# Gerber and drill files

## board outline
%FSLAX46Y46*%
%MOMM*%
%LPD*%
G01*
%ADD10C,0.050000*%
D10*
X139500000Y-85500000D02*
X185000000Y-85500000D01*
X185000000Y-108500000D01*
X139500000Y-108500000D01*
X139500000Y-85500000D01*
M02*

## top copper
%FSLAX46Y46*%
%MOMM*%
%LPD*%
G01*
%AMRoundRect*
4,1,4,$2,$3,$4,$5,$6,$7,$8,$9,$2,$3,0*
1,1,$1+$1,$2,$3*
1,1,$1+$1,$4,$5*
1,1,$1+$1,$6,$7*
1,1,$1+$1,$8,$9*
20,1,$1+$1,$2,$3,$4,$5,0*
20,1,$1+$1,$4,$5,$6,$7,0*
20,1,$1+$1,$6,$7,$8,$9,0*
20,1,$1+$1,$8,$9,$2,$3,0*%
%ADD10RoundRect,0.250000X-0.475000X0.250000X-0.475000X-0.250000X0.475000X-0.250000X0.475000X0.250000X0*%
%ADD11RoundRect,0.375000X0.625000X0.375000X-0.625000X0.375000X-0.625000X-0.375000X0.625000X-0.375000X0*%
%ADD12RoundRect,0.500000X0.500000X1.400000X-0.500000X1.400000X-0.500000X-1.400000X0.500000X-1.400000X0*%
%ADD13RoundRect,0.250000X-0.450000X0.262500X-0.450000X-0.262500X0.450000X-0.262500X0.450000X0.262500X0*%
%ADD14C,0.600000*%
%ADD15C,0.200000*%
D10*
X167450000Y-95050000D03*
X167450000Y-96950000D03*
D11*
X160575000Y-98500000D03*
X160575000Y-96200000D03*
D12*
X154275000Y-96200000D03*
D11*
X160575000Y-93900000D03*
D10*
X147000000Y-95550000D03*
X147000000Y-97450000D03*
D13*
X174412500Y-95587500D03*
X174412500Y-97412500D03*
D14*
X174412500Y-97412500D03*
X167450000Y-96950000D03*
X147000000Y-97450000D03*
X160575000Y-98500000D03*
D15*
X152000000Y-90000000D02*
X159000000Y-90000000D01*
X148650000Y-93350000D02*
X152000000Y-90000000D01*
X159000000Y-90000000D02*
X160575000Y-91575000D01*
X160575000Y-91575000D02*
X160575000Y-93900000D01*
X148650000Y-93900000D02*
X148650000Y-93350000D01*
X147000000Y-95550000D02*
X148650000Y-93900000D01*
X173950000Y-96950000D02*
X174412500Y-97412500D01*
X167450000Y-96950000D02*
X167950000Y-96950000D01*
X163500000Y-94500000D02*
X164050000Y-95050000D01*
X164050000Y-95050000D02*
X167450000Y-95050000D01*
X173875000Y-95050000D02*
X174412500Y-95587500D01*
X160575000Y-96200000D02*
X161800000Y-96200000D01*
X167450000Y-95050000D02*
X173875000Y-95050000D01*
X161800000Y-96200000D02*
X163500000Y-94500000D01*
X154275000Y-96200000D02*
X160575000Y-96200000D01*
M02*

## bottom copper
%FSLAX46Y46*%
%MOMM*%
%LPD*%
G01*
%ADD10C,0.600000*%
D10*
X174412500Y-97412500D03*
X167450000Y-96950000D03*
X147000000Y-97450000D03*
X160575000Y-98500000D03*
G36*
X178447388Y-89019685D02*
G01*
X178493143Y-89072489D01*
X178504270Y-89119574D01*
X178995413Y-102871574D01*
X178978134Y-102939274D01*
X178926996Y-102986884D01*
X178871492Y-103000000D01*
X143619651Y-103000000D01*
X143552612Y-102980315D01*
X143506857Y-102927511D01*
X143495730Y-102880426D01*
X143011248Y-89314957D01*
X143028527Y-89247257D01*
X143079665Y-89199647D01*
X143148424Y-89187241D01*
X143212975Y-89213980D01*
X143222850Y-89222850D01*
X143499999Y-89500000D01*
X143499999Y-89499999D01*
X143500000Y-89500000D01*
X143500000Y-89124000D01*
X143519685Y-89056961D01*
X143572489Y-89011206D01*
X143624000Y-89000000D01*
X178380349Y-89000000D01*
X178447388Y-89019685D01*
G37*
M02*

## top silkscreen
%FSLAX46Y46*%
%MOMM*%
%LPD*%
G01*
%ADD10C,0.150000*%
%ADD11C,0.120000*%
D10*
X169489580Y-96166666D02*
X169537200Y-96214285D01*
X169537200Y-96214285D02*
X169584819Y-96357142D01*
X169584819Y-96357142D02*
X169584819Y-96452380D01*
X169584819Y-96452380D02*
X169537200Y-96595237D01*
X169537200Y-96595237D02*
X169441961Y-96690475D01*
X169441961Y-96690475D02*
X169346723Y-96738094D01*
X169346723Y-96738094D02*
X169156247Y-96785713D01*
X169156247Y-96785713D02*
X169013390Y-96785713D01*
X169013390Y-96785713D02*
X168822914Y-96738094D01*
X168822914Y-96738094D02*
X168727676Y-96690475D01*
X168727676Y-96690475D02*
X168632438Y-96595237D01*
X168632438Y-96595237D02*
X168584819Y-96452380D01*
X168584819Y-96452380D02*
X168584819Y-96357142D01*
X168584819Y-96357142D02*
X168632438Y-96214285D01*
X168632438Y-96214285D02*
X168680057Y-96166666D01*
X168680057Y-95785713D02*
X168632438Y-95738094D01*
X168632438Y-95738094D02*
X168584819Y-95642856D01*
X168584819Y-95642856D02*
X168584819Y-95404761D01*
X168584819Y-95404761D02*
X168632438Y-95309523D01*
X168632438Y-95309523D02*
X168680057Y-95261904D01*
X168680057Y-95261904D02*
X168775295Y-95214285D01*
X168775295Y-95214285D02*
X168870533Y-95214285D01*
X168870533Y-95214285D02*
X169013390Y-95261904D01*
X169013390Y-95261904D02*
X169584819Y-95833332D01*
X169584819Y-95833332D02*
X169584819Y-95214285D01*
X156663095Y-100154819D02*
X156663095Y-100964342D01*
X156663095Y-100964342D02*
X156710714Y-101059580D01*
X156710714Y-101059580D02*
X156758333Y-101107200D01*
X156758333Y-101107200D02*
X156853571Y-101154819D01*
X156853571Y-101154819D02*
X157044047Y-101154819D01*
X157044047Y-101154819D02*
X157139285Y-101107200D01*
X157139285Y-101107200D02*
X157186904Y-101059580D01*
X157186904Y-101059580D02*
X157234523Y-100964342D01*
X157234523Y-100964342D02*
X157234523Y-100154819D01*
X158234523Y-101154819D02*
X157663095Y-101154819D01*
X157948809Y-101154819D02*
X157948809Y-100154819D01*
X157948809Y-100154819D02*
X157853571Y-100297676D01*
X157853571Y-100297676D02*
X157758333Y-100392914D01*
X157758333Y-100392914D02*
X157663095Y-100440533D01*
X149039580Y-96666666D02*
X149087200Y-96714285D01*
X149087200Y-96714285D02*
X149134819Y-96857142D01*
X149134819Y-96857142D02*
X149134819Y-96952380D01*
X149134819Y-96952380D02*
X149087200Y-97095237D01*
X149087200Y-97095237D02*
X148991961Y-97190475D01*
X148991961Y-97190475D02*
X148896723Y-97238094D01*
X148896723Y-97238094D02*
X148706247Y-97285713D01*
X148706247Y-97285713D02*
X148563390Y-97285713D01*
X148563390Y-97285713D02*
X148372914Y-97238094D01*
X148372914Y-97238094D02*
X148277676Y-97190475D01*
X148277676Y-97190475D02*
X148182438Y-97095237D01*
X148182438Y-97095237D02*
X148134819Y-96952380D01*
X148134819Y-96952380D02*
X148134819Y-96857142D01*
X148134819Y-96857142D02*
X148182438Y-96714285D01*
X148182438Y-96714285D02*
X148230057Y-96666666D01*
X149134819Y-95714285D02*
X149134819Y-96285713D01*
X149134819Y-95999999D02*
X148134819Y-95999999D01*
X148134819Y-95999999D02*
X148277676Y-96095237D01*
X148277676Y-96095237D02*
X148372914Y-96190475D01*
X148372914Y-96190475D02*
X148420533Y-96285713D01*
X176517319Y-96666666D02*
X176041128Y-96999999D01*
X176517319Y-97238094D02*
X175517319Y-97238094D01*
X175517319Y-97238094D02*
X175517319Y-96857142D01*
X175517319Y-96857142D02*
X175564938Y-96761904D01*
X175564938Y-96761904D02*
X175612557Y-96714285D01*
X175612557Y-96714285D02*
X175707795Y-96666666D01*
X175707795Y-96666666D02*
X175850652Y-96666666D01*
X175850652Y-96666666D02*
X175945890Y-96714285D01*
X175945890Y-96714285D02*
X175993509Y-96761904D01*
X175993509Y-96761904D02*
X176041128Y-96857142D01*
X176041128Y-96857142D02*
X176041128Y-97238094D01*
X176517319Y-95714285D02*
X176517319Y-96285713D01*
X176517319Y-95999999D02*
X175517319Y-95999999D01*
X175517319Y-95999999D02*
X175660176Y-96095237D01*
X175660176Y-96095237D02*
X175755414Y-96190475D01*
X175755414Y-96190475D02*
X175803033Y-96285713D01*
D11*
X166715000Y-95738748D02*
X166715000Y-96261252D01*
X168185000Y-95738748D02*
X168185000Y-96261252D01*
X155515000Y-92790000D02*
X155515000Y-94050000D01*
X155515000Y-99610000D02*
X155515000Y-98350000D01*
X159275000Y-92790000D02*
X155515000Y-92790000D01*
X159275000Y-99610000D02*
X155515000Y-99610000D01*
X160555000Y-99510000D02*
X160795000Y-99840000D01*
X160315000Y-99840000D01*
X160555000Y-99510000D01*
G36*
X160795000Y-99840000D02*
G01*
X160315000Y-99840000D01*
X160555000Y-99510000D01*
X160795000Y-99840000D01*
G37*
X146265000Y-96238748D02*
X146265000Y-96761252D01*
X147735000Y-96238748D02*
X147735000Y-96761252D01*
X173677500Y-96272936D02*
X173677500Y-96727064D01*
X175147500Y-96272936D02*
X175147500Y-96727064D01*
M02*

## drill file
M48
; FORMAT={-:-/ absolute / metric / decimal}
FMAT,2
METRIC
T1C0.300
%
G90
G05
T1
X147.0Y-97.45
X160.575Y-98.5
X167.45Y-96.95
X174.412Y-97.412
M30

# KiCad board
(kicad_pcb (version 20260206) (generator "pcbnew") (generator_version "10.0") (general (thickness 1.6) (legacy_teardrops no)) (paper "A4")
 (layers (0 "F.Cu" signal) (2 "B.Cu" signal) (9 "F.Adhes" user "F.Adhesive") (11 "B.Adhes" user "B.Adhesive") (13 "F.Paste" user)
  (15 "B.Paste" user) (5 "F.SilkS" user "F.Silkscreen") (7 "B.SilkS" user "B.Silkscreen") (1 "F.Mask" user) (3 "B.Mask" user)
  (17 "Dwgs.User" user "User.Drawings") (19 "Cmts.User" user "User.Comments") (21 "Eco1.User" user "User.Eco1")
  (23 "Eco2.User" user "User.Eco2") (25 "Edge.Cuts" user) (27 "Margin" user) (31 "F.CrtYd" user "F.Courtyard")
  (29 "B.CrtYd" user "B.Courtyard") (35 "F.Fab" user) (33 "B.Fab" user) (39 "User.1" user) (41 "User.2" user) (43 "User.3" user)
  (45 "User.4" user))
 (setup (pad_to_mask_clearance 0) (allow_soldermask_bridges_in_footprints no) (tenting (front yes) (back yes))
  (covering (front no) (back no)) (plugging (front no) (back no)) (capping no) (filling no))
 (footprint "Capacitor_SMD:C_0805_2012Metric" (layer "F.Cu") (at 167.45 96 -90)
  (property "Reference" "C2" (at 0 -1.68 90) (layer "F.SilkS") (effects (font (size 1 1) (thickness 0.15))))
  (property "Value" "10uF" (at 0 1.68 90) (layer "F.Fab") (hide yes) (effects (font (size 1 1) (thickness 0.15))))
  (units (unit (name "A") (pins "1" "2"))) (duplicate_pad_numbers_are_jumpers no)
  (fp_line (start -0.261252 0.735) (end 0.261252 0.735) (stroke (width 0.12) (type solid)) (layer "F.SilkS"))
  (fp_line (start -0.261252 -0.735) (end 0.261252 -0.735) (stroke (width 0.12) (type solid)) (layer "F.SilkS"))
  (pad "1" smd roundrect (at -0.95 0 270) (size 1 1.45) (layers "F.Cu" "F.Mask" "F.Paste") (roundrect_rratio 0.25) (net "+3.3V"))
  (pad "2" smd roundrect (at 0.95 0 270) (size 1 1.45) (layers "F.Cu" "F.Mask" "F.Paste") (roundrect_rratio 0.25) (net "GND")))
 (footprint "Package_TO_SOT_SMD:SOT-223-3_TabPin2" (layer "F.Cu") (at 157.425 96.2 180)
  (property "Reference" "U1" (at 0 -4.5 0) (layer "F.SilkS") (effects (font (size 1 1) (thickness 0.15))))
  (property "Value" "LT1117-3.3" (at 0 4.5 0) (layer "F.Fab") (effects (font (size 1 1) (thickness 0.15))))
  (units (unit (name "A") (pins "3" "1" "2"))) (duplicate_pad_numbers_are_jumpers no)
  (fp_line (start 1.91 3.41) (end 1.91 2.15) (stroke (width 0.12) (type solid)) (layer "F.SilkS"))
  (fp_line (start 1.91 -3.41) (end 1.91 -2.15) (stroke (width 0.12) (type solid)) (layer "F.SilkS"))
  (fp_line (start -1.85 3.41) (end 1.91 3.41) (stroke (width 0.12) (type solid)) (layer "F.SilkS"))
  (fp_line (start -1.85 -3.41) (end 1.91 -3.41) (stroke (width 0.12) (type solid)) (layer "F.SilkS"))
  (fp_poly
   (pts (xy -3.13 -3.31) (xy -3.37 -3.64) (xy -2.89 -3.64) (xy -3.13 -3.31)) (stroke (width 0.12) (type solid)) (fill yes) (layer "F.SilkS"))
  (pad "1" smd roundrect (at -3.15 -2.3 180) (size 2 1.5) (layers "F.Cu" "F.Mask" "F.Paste") (roundrect_rratio 0.25) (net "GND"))
  (pad "2" smd roundrect (at -3.15 0 180) (size 2 1.5) (layers "F.Cu" "F.Mask" "F.Paste") (roundrect_rratio 0.25) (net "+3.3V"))
  (pad "2" smd roundrect (at 3.15 0 180) (size 2 3.8) (layers "F.Cu" "F.Mask" "F.Paste") (roundrect_rratio 0.25) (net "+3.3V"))
  (pad "3" smd roundrect (at -3.15 2.3 180) (size 2 1.5) (layers "F.Cu" "F.Mask" "F.Paste") (roundrect_rratio 0.25) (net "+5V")))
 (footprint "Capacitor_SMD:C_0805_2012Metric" (layer "F.Cu") (at 147 96.5 -90)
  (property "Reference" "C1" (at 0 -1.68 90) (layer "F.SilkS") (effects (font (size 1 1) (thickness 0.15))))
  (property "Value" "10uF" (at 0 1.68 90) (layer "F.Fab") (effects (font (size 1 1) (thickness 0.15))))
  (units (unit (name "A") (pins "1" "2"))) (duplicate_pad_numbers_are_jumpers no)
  (fp_line (start -0.261252 0.735) (end 0.261252 0.735) (stroke (width 0.12) (type solid)) (layer "F.SilkS"))
  (fp_line (start -0.261252 -0.735) (end 0.261252 -0.735) (stroke (width 0.12) (type solid)) (layer "F.SilkS"))
  (pad "1" smd roundrect (at -0.95 0 270) (size 1 1.45) (layers "F.Cu" "F.Mask" "F.Paste") (roundrect_rratio 0.25) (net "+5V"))
  (pad "2" smd roundrect (at 0.95 0 270) (size 1 1.45) (layers "F.Cu" "F.Mask" "F.Paste") (roundrect_rratio 0.25) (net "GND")))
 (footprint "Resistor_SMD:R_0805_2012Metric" (layer "F.Cu") (at 174.4125 96.5 -90)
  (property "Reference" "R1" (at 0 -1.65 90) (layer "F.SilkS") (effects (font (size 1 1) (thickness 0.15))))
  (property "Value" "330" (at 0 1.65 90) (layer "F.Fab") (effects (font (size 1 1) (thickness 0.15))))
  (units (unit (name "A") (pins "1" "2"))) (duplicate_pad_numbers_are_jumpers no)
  (fp_line (start -0.227064 0.735) (end 0.227064 0.735) (stroke (width 0.12) (type solid)) (layer "F.SilkS"))
  (fp_line (start -0.227064 -0.735) (end 0.227064 -0.735) (stroke (width 0.12) (type solid)) (layer "F.SilkS"))
  (pad "1" smd roundrect (at -0.9125 0 270) (size 1.025 1.4) (layers "F.Cu" "F.Mask" "F.Paste") (roundrect_rratio 0.243902) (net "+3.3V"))
  (pad "2" smd roundrect (at 0.9125 0 270) (size 1.025 1.4) (layers "F.Cu" "F.Mask" "F.Paste") (roundrect_rratio 0.243902) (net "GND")))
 (gr_rect (start 139.5 85.5) (end 185 108.5) (stroke (width 0.05) (type default)) (fill no) (layer "Edge.Cuts"))
 (segment (start 152 90) (end 159 90) (width 0.2) (layer "F.Cu") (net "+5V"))
 (segment (start 148.65 93.35) (end 152 90) (width 0.2) (layer "F.Cu") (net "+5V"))
 (segment (start 159 90) (end 160.575 91.575) (width 0.2) (layer "F.Cu") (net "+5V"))
 (segment (start 160.575 91.575) (end 160.575 93.9) (width 0.2) (layer "F.Cu") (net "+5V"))
 (segment (start 148.65 93.9) (end 148.65 93.35) (width 0.2) (layer "F.Cu") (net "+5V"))
 (segment (start 147 95.55) (end 148.65 93.9) (width 0.2) (layer "F.Cu") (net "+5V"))
 (segment (start 173.95 96.95) (end 174.4125 97.4125) (width 0.2) (layer "F.Cu") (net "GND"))
 (segment (start 167.45 96.95) (end 167.95 96.95) (width 0.2) (layer "F.Cu") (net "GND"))
 (via (at 174.4125 97.4125) (size 0.6) (drill 0.3) (layers "F.Cu" "B.Cu") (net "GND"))
 (via (at 167.45 96.95) (size 0.6) (drill 0.3) (layers "F.Cu" "B.Cu") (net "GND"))
 (via (at 147 97.45) (size 0.6) (drill 0.3) (layers "F.Cu" "B.Cu") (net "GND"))
 (via (at 160.575 98.5) (size 0.6) (drill 0.3) (layers "F.Cu" "B.Cu") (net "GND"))
 (segment (start 163.5 94.5) (end 164.05 95.05) (width 0.2) (layer "F.Cu") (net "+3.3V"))
 (segment (start 164.05 95.05) (end 167.45 95.05) (width 0.2) (layer "F.Cu") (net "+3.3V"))
 (segment (start 173.875 95.05) (end 174.4125 95.5875) (width 0.2) (layer "F.Cu") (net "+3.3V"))
 (segment (start 160.575 96.2) (end 161.8 96.2) (width 0.2) (layer "F.Cu") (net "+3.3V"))
 (segment (start 167.45 95.05) (end 173.875 95.05) (width 0.2) (layer "F.Cu") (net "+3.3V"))
 (segment (start 161.8 96.2) (end 163.5 94.5) (width 0.2) (layer "F.Cu") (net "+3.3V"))
 (segment (start 154.275 96.2) (end 160.575 96.2) (width 0.2) (layer "F.Cu") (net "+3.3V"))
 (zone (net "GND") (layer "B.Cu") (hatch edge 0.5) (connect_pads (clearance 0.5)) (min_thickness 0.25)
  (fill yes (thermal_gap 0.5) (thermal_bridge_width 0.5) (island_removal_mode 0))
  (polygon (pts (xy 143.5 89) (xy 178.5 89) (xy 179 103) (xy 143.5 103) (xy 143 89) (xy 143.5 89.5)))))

